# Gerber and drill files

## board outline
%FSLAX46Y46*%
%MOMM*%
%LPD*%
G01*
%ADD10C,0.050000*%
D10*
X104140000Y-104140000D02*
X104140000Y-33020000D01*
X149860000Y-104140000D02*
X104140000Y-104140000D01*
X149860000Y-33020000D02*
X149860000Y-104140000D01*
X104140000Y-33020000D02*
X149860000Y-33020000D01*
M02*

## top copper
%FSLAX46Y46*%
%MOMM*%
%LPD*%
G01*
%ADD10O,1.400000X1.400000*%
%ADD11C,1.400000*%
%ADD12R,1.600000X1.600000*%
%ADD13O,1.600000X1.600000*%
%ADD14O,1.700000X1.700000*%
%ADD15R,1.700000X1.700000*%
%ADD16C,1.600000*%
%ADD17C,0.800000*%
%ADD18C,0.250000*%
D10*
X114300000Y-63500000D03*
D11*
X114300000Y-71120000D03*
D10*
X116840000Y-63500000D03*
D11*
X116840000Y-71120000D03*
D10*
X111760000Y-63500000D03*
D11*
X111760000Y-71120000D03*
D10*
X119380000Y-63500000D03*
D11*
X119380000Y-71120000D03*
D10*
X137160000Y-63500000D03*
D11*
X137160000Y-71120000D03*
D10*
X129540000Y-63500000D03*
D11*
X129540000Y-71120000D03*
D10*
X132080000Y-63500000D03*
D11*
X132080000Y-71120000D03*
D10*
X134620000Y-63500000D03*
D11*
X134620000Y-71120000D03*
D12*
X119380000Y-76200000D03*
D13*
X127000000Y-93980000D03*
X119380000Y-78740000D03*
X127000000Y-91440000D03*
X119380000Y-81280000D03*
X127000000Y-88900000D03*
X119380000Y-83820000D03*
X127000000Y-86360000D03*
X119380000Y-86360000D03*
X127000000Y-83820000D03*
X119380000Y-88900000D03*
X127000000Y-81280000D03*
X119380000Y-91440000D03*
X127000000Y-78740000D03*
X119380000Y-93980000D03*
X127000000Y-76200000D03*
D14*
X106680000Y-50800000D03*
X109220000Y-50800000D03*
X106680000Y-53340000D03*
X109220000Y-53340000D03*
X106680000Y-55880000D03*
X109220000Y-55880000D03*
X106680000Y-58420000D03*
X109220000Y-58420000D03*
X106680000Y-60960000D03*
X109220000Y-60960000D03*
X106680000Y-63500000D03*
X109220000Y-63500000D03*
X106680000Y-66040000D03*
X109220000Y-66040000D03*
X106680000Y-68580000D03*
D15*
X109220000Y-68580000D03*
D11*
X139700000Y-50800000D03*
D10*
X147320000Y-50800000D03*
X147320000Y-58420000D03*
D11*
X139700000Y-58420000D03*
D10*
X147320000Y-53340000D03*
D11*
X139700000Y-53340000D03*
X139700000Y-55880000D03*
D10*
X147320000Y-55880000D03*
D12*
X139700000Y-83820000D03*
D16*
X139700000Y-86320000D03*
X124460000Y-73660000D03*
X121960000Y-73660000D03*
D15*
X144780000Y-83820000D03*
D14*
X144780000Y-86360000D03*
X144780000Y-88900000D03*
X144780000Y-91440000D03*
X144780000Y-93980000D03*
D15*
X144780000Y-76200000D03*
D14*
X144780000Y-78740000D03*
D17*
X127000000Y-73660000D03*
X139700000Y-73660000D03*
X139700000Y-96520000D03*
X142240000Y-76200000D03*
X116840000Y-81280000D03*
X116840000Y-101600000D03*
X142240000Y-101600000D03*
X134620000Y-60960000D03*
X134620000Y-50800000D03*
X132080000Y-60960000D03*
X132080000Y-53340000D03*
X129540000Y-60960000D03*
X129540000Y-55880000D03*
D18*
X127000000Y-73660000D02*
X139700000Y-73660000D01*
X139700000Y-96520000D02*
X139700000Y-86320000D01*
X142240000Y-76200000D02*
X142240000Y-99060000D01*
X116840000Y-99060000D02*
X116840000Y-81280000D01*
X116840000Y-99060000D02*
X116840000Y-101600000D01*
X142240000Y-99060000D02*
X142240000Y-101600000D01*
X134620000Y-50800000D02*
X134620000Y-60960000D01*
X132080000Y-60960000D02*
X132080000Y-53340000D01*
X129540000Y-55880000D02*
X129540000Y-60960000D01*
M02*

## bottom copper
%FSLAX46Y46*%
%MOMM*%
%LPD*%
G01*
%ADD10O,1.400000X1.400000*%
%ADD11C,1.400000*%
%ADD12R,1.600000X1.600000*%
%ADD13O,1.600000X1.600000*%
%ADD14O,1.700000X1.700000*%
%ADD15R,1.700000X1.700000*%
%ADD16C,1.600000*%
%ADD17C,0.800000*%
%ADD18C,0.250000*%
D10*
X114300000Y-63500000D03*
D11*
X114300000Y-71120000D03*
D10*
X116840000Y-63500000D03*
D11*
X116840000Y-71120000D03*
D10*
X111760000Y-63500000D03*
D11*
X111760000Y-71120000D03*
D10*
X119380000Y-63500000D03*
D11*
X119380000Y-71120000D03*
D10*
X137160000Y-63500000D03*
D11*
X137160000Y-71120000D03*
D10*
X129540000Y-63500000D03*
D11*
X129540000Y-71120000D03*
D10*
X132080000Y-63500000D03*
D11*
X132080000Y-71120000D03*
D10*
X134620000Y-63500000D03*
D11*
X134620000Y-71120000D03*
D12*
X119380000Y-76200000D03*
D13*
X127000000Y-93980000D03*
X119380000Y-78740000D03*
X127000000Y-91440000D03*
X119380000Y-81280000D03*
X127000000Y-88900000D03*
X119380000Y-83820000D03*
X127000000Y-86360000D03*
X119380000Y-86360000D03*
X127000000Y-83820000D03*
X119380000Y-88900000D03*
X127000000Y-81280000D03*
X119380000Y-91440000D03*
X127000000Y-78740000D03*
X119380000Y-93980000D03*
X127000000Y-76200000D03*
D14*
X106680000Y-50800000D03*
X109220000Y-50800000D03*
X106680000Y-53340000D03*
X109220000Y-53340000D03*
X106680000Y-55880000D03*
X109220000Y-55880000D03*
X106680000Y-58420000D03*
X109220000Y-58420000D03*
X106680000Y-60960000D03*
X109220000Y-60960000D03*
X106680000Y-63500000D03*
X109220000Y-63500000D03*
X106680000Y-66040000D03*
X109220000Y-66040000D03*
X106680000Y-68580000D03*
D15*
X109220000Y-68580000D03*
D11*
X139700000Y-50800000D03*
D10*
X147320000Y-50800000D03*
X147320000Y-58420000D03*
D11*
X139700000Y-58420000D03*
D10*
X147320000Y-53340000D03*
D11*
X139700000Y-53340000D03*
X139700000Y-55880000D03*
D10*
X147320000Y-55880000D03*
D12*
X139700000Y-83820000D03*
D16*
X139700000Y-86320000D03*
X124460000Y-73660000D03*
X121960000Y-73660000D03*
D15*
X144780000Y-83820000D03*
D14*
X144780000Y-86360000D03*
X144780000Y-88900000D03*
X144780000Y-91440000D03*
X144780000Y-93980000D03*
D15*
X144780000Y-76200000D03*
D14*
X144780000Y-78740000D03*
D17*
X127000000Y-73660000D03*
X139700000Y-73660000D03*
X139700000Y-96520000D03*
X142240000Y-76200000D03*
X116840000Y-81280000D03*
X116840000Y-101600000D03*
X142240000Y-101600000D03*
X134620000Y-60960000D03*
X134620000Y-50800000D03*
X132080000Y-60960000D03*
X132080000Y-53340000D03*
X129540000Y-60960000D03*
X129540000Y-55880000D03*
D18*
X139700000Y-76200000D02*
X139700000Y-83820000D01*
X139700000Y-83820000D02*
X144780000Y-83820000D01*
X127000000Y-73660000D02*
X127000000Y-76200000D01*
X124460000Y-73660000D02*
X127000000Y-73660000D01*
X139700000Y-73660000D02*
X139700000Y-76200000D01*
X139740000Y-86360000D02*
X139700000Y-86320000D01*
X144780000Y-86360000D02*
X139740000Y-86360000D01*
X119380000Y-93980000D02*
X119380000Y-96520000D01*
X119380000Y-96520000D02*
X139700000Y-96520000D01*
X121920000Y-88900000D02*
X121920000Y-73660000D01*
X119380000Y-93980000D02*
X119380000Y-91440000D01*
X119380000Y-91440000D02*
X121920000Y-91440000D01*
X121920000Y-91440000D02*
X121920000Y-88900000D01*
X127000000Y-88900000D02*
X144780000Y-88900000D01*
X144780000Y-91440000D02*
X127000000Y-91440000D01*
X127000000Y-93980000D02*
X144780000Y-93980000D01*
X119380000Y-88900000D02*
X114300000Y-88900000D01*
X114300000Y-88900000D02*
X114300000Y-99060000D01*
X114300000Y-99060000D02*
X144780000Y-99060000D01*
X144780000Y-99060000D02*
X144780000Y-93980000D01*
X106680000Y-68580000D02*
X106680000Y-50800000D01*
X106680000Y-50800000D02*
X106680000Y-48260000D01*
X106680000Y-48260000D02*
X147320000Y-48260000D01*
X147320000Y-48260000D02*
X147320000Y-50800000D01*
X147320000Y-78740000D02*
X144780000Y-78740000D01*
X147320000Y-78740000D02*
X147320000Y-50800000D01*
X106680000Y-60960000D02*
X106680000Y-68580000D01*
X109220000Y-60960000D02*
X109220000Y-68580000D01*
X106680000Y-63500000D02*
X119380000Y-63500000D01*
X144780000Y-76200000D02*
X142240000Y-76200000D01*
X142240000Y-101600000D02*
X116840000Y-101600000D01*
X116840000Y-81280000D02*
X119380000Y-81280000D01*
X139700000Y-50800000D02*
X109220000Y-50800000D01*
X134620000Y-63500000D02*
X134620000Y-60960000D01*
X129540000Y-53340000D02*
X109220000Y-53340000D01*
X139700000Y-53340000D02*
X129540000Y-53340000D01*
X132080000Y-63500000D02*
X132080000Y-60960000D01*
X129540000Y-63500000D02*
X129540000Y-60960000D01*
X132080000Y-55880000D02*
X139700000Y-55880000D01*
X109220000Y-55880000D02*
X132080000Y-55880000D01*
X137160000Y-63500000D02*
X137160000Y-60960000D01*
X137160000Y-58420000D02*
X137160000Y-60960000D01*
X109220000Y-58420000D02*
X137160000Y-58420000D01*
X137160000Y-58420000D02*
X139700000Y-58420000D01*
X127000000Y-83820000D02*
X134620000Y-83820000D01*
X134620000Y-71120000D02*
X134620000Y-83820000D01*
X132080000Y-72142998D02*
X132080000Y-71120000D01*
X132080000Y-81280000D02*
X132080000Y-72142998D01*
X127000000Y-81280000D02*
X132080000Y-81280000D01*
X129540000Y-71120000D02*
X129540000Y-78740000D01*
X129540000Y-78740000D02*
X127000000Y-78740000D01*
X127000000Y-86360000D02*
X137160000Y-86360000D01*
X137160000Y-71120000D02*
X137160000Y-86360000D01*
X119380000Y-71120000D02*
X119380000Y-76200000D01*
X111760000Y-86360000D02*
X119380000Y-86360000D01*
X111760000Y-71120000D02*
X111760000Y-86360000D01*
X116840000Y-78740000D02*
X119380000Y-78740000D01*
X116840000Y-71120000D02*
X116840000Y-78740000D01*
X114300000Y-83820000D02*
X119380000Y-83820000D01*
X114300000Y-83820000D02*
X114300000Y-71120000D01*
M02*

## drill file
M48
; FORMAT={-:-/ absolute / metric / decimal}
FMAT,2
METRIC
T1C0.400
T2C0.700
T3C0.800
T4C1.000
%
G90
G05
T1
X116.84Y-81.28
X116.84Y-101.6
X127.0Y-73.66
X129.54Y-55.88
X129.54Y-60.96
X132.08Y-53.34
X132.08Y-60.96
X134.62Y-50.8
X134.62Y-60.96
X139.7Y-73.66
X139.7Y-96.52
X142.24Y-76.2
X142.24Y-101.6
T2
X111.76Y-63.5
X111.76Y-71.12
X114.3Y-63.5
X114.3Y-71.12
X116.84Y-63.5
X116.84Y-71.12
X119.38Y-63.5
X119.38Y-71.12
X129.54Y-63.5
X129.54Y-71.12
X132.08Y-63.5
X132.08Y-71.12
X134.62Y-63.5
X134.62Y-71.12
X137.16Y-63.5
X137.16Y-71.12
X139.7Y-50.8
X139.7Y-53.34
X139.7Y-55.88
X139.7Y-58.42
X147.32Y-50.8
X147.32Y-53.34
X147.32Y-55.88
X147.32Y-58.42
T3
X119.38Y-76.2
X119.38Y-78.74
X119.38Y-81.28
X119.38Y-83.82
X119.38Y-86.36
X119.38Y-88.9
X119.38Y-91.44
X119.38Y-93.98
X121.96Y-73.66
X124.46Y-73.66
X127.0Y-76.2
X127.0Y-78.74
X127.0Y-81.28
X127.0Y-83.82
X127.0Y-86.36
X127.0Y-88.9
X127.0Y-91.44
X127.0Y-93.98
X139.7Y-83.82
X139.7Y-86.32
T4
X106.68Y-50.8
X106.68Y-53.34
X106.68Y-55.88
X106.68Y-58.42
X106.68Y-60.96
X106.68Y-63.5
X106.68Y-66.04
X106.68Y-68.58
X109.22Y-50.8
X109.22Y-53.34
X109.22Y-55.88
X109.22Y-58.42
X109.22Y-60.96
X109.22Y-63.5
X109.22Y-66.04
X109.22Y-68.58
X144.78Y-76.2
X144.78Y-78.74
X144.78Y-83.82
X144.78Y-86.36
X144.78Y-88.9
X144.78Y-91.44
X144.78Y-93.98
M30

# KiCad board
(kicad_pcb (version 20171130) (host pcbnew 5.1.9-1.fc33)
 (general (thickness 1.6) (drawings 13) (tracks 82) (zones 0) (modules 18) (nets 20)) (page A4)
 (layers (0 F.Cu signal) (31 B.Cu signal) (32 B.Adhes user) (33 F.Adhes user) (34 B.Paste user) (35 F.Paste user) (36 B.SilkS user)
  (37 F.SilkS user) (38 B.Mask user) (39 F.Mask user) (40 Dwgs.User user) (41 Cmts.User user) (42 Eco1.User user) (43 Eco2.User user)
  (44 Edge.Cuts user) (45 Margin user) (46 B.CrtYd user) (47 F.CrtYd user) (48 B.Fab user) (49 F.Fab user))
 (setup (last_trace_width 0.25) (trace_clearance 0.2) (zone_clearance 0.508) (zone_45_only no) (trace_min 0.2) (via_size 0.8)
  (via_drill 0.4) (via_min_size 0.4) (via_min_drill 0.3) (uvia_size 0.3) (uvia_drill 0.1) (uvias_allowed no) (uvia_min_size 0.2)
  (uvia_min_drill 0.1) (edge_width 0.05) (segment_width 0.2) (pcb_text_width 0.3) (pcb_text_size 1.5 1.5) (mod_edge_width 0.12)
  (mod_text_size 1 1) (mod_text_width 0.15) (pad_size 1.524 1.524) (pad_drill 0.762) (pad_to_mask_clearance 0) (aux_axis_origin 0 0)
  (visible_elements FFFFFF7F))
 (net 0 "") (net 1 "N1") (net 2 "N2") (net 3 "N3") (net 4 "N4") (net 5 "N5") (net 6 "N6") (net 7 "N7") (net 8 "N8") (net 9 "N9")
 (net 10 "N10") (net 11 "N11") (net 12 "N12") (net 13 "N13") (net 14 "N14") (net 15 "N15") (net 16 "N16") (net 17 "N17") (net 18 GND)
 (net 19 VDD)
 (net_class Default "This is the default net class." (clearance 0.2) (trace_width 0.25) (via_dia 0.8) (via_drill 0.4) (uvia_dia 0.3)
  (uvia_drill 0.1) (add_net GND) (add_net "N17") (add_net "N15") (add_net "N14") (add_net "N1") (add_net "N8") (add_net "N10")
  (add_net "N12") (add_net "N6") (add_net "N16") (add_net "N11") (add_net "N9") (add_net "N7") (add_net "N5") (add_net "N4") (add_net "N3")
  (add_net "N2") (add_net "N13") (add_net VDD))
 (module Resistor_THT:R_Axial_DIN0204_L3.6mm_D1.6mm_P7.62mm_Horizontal (layer F.Cu) (at 114.3 71.12 90)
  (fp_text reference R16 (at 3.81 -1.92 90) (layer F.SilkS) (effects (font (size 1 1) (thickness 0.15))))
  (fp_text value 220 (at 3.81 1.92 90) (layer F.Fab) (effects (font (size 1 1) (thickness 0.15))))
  (pad 2 thru_hole oval (at 7.62 0 90) (size 1.4 1.4) (drill 0.7) (layers *.Cu *.Mask) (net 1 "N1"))
  (pad 1 thru_hole circle (at 0 0 90) (size 1.4 1.4) (drill 0.7) (layers *.Cu *.Mask) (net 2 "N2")))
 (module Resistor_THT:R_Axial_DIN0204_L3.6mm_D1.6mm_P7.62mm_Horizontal (layer F.Cu) (at 116.84 71.12 90)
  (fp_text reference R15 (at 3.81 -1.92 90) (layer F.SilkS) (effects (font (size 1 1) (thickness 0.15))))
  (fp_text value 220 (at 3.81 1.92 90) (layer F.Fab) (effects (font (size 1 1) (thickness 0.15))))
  (pad 2 thru_hole oval (at 7.62 0 90) (size 1.4 1.4) (drill 0.7) (layers *.Cu *.Mask) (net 1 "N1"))
  (pad 1 thru_hole circle (at 0 0 90) (size 1.4 1.4) (drill 0.7) (layers *.Cu *.Mask) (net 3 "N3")))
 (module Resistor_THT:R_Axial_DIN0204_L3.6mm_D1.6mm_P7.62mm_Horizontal (layer F.Cu) (at 111.76 71.12 90)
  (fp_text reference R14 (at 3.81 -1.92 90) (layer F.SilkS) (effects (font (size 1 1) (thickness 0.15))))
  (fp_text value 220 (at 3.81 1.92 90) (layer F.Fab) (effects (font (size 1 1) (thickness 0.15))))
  (pad 2 thru_hole oval (at 7.62 0 90) (size 1.4 1.4) (drill 0.7) (layers *.Cu *.Mask) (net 1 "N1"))
  (pad 1 thru_hole circle (at 0 0 90) (size 1.4 1.4) (drill 0.7) (layers *.Cu *.Mask) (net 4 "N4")))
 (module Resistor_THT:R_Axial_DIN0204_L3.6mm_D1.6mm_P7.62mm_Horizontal (layer F.Cu) (at 119.38 71.12 90)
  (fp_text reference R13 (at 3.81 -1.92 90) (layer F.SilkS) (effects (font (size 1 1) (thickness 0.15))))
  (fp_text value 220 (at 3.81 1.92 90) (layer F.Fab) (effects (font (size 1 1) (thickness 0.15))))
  (pad 2 thru_hole oval (at 7.62 0 90) (size 1.4 1.4) (drill 0.7) (layers *.Cu *.Mask) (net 1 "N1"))
  (pad 1 thru_hole circle (at 0 0 90) (size 1.4 1.4) (drill 0.7) (layers *.Cu *.Mask) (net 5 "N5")))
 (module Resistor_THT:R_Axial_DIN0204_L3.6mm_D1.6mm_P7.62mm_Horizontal (layer F.Cu) (at 137.16 71.12 90)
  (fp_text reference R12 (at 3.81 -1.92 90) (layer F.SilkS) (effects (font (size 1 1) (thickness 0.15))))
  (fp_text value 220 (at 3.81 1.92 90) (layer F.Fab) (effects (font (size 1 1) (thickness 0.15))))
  (pad 2 thru_hole oval (at 7.62 0 90) (size 1.4 1.4) (drill 0.7) (layers *.Cu *.Mask) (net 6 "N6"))
  (pad 1 thru_hole circle (at 0 0 90) (size 1.4 1.4) (drill 0.7) (layers *.Cu *.Mask) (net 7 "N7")))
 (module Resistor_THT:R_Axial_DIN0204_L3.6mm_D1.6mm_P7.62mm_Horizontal (layer F.Cu) (at 129.54 71.12 90)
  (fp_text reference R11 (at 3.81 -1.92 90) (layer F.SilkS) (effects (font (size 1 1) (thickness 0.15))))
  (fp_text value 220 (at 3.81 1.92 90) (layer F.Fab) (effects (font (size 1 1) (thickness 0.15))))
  (pad 2 thru_hole oval (at 7.62 0 90) (size 1.4 1.4) (drill 0.7) (layers *.Cu *.Mask) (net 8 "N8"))
  (pad 1 thru_hole circle (at 0 0 90) (size 1.4 1.4) (drill 0.7) (layers *.Cu *.Mask) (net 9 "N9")))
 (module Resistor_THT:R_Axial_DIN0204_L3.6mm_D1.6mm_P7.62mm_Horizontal (layer F.Cu) (at 132.08 71.12 90)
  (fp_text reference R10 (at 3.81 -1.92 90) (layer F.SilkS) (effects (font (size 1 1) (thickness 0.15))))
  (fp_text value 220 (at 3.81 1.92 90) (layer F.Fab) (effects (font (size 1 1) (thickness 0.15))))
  (pad 2 thru_hole oval (at 7.62 0 90) (size 1.4 1.4) (drill 0.7) (layers *.Cu *.Mask) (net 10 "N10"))
  (pad 1 thru_hole circle (at 0 0 90) (size 1.4 1.4) (drill 0.7) (layers *.Cu *.Mask) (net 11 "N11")))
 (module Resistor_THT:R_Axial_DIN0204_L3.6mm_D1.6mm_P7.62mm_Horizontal (layer F.Cu) (at 134.62 71.12 90)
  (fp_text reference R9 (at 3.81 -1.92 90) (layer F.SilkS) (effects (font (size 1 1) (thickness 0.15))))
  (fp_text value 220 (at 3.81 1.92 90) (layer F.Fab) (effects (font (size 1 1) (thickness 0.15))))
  (pad 2 thru_hole oval (at 7.62 0 90) (size 1.4 1.4) (drill 0.7) (layers *.Cu *.Mask) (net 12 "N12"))
  (pad 1 thru_hole circle (at 0 0 90) (size 1.4 1.4) (drill 0.7) (layers *.Cu *.Mask) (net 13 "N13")))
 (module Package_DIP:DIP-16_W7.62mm (layer F.Cu) (at 119.38 76.2)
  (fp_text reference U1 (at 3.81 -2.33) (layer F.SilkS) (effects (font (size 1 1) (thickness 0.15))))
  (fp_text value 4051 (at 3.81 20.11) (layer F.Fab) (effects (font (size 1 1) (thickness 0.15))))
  (pad 1 thru_hole rect (at 0 0) (size 1.6 1.6) (drill 0.8) (layers *.Cu *.Mask) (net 5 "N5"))
  (pad 9 thru_hole oval (at 7.62 17.78) (size 1.6 1.6) (drill 0.8) (layers *.Cu *.Mask) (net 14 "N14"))
  (pad 2 thru_hole oval (at 0 2.54) (size 1.6 1.6) (drill 0.8) (layers *.Cu *.Mask) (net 3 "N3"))
  (pad 10 thru_hole oval (at 7.62 15.24) (size 1.6 1.6) (drill 0.8) (layers *.Cu *.Mask) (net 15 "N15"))
  (pad 3 thru_hole oval (at 0 5.08) (size 1.6 1.6) (drill 0.8) (layers *.Cu *.Mask) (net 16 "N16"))
  (pad 11 thru_hole oval (at 7.62 12.7) (size 1.6 1.6) (drill 0.8) (layers *.Cu *.Mask) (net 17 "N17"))
  (pad 4 thru_hole oval (at 0 7.62) (size 1.6 1.6) (drill 0.8) (layers *.Cu *.Mask) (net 2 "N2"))
  (pad 12 thru_hole oval (at 7.62 10.16) (size 1.6 1.6) (drill 0.8) (layers *.Cu *.Mask) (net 7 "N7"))
  (pad 5 thru_hole oval (at 0 10.16) (size 1.6 1.6) (drill 0.8) (layers *.Cu *.Mask) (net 4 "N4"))
  (pad 13 thru_hole oval (at 7.62 7.62) (size 1.6 1.6) (drill 0.8) (layers *.Cu *.Mask) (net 13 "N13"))
  (pad 6 thru_hole oval (at 0 12.7) (size 1.6 1.6) (drill 0.8) (layers *.Cu *.Mask) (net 14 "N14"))
  (pad 14 thru_hole oval (at 7.62 5.08) (size 1.6 1.6) (drill 0.8) (layers *.Cu *.Mask) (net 11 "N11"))
  (pad 7 thru_hole oval (at 0 15.24) (size 1.6 1.6) (drill 0.8) (layers *.Cu *.Mask) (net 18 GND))
  (pad 15 thru_hole oval (at 7.62 2.54) (size 1.6 1.6) (drill 0.8) (layers *.Cu *.Mask) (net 9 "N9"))
  (pad 8 thru_hole oval (at 0 17.78) (size 1.6 1.6) (drill 0.8) (layers *.Cu *.Mask) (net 18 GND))
  (pad 16 thru_hole oval (at 7.62 0) (size 1.6 1.6) (drill 0.8) (layers *.Cu *.Mask) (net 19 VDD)))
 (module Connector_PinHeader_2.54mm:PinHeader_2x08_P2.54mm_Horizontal (layer F.Cu) (at 109.22 68.58 180)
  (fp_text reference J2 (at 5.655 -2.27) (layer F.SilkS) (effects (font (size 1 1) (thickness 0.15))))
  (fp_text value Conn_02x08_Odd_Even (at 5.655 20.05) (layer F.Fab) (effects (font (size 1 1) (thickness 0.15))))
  (pad 16 thru_hole oval (at 2.54 17.78 180) (size 1.7 1.7) (drill 1) (layers *.Cu *.Mask) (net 1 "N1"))
  (pad 15 thru_hole oval (at 0 17.78 180) (size 1.7 1.7) (drill 1) (layers *.Cu *.Mask) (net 12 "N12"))
  (pad 14 thru_hole oval (at 2.54 15.24 180) (size 1.7 1.7) (drill 1) (layers *.Cu *.Mask) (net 1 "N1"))
  (pad 13 thru_hole oval (at 0 15.24 180) (size 1.7 1.7) (drill 1) (layers *.Cu *.Mask) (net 10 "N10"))
  (pad 12 thru_hole oval (at 2.54 12.7 180) (size 1.7 1.7) (drill 1) (layers *.Cu *.Mask) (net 1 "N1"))
  (pad 11 thru_hole oval (at 0 12.7 180) (size 1.7 1.7) (drill 1) (layers *.Cu *.Mask) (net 8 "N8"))
  (pad 10 thru_hole oval (at 2.54 10.16 180) (size 1.7 1.7) (drill 1) (layers *.Cu *.Mask) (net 1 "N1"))
  (pad 9 thru_hole oval (at 0 10.16 180) (size 1.7 1.7) (drill 1) (layers *.Cu *.Mask) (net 6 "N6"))
  (pad 8 thru_hole oval (at 2.54 7.62 180) (size 1.7 1.7) (drill 1) (layers *.Cu *.Mask) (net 1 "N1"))
  (pad 7 thru_hole oval (at 0 7.62 180) (size 1.7 1.7) (drill 1) (layers *.Cu *.Mask) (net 1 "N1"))
  (pad 6 thru_hole oval (at 2.54 5.08 180) (size 1.7 1.7) (drill 1) (layers *.Cu *.Mask) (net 1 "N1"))
  (pad 5 thru_hole oval (at 0 5.08 180) (size 1.7 1.7) (drill 1) (layers *.Cu *.Mask) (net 1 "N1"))
  (pad 4 thru_hole oval (at 2.54 2.54 180) (size 1.7 1.7) (drill 1) (layers *.Cu *.Mask) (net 1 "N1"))
  (pad 3 thru_hole oval (at 0 2.54 180) (size 1.7 1.7) (drill 1) (layers *.Cu *.Mask) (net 1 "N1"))
  (pad 2 thru_hole oval (at 2.54 0 180) (size 1.7 1.7) (drill 1) (layers *.Cu *.Mask) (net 1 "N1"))
  (pad 1 thru_hole rect (at 0 0 180) (size 1.7 1.7) (drill 1) (layers *.Cu *.Mask) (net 1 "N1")))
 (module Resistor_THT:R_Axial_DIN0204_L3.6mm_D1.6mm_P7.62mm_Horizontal (layer F.Cu) (at 139.7 50.8)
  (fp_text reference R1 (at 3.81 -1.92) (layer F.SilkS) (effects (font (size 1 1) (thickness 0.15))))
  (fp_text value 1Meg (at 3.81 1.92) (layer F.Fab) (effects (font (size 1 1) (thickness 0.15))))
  (pad 1 thru_hole circle (at 0 0) (size 1.4 1.4) (drill 0.7) (layers *.Cu *.Mask) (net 12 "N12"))
  (pad 2 thru_hole oval (at 7.62 0) (size 1.4 1.4) (drill 0.7) (layers *.Cu *.Mask) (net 1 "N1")))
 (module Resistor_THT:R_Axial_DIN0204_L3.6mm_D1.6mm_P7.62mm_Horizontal (layer F.Cu) (at 139.7 58.42)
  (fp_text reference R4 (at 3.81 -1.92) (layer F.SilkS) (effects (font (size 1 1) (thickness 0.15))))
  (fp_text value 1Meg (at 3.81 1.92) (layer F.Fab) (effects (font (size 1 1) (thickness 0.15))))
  (pad 2 thru_hole oval (at 7.62 0) (size 1.4 1.4) (drill 0.7) (layers *.Cu *.Mask) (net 1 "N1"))
  (pad 1 thru_hole circle (at 0 0) (size 1.4 1.4) (drill 0.7) (layers *.Cu *.Mask) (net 6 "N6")))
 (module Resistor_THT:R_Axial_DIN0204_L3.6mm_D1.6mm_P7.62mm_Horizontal (layer F.Cu) (at 139.7 53.34)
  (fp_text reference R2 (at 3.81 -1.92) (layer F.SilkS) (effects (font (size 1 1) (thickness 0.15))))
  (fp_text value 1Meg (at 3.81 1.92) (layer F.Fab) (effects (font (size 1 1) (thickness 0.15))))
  (pad 2 thru_hole oval (at 7.62 0) (size 1.4 1.4) (drill 0.7) (layers *.Cu *.Mask) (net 1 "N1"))
  (pad 1 thru_hole circle (at 0 0) (size 1.4 1.4) (drill 0.7) (layers *.Cu *.Mask) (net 10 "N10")))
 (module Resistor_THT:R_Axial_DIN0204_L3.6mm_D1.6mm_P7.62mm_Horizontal (layer F.Cu) (at 139.7 55.88)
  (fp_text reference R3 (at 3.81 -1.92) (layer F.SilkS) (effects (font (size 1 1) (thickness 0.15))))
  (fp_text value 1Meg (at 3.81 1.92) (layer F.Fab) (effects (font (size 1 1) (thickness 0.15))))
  (pad 1 thru_hole circle (at 0 0) (size 1.4 1.4) (drill 0.7) (layers *.Cu *.Mask) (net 8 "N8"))
  (pad 2 thru_hole oval (at 7.62 0) (size 1.4 1.4) (drill 0.7) (layers *.Cu *.Mask) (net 1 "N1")))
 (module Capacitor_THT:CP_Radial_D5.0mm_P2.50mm (layer F.Cu) (at 139.7 83.82 270)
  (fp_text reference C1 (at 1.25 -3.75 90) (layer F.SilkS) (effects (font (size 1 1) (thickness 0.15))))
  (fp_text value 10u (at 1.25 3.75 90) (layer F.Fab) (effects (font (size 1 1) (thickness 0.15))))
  (pad 1 thru_hole rect (at 0 0 270) (size 1.6 1.6) (drill 0.8) (layers *.Cu *.Mask) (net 19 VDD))
  (pad 2 thru_hole circle (at 2.5 0 270) (size 1.6 1.6) (drill 0.8) (layers *.Cu *.Mask) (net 18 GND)))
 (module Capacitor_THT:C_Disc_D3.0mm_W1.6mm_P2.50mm (layer F.Cu) (at 124.46 73.66 180)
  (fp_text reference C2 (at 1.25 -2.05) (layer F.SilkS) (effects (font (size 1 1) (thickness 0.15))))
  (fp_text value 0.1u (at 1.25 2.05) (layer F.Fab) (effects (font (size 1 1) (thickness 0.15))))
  (pad 1 thru_hole circle (at 0 0 180) (size 1.6 1.6) (drill 0.8) (layers *.Cu *.Mask) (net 19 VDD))
  (pad 2 thru_hole circle (at 2.5 0 180) (size 1.6 1.6) (drill 0.8) (layers *.Cu *.Mask) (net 18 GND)))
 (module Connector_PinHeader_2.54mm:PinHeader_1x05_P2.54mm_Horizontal (layer F.Cu) (at 144.78 83.82)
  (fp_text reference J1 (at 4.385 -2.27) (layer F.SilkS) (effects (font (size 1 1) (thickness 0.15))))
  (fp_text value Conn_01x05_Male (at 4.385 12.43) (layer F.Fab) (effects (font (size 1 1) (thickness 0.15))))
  (pad 1 thru_hole rect (at 0 0) (size 1.7 1.7) (drill 1) (layers *.Cu *.Mask) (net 19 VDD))
  (pad 2 thru_hole oval (at 0 2.54) (size 1.7 1.7) (drill 1) (layers *.Cu *.Mask) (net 18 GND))
  (pad 3 thru_hole oval (at 0 5.08) (size 1.7 1.7) (drill 1) (layers *.Cu *.Mask) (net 17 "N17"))
  (pad 4 thru_hole oval (at 0 7.62) (size 1.7 1.7) (drill 1) (layers *.Cu *.Mask) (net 15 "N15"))
  (pad 5 thru_hole oval (at 0 10.16) (size 1.7 1.7) (drill 1) (layers *.Cu *.Mask) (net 14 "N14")))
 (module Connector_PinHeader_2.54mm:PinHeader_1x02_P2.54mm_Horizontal (layer F.Cu) (at 144.78 76.2)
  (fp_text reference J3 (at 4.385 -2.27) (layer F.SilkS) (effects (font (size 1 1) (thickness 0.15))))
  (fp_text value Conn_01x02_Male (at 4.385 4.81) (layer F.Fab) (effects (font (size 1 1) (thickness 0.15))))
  (pad 1 thru_hole rect (at 0 0) (size 1.7 1.7) (drill 1) (layers *.Cu *.Mask) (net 16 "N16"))
  (pad 2 thru_hole oval (at 0 2.54) (size 1.7 1.7) (drill 1) (layers *.Cu *.Mask) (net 1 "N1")))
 (gr_line (start 104.14 104.14) (end 104.14 33.02) (layer Edge.Cuts) (width 0.05))
 (gr_line (start 149.86 104.14) (end 104.14 104.14) (layer Edge.Cuts) (width 0.05))
 (gr_line (start 149.86 33.02) (end 149.86 104.14) (layer Edge.Cuts) (width 0.05))
 (gr_line (start 104.14 33.02) (end 149.86 33.02) (layer Edge.Cuts) (width 0.05))
 (segment (start 139.7 76.2) (end 139.7 83.82) (width 0.25) (layer B.Cu) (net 19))
 (segment (start 139.7 83.82) (end 144.78 83.82) (width 0.25) (layer B.Cu) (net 19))
 (segment (start 127 73.66) (end 127 76.2) (width 0.25) (layer B.Cu) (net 19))
 (via (at 127 73.66) (size 0.8) (drill 0.4) (layers F.Cu B.Cu) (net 19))
 (segment (start 124.46 73.66) (end 127 73.66) (width 0.25) (layer B.Cu) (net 19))
 (via (at 139.7 73.66) (size 0.8) (drill 0.4) (layers F.Cu B.Cu) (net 19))
 (segment (start 127 73.66) (end 139.7 73.66) (width 0.25) (layer F.Cu) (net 19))
 (segment (start 139.7 73.66) (end 139.7 76.2) (width 0.25) (layer B.Cu) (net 19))
 (segment (start 139.74 86.36) (end 139.7 86.32) (width 0.25) (layer B.Cu) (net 18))
 (segment (start 144.78 86.36) (end 139.74 86.36) (width 0.25) (layer B.Cu) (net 18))
 (segment (start 119.38 93.98) (end 119.38 96.52) (width 0.25) (layer B.Cu) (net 18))
 (via (at 139.7 96.52) (size 0.8) (drill 0.4) (layers F.Cu B.Cu) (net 18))
 (segment (start 119.38 96.52) (end 139.7 96.52) (width 0.25) (layer B.Cu) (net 18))
 (segment (start 139.7 96.52) (end 139.7 86.32) (width 0.25) (layer F.Cu) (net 18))
 (segment (start 121.92 88.9) (end 121.92 73.66) (width 0.25) (layer B.Cu) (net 18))
 (segment (start 119.38 93.98) (end 119.38 91.44) (width 0.25) (layer B.Cu) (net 18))
 (segment (start 119.38 91.44) (end 121.92 91.44) (width 0.25) (layer B.Cu) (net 18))
 (segment (start 121.92 91.44) (end 121.92 88.9) (width 0.25) (layer B.Cu) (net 18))
 (segment (start 127 88.9) (end 144.78 88.9) (width 0.25) (layer B.Cu) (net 17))
 (segment (start 144.78 91.44) (end 127 91.44) (width 0.25) (layer B.Cu) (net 15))
 (segment (start 127 93.98) (end 144.78 93.98) (width 0.25) (layer B.Cu) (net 14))
 (segment (start 119.38 88.9) (end 114.3 88.9) (width 0.25) (layer B.Cu) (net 14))
 (segment (start 114.3 88.9) (end 114.3 99.06) (width 0.25) (layer B.Cu) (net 14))
 (segment (start 114.3 99.06) (end 144.78 99.06) (width 0.25) (layer B.Cu) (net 14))
 (segment (start 144.78 99.06) (end 144.78 93.98) (width 0.25) (layer B.Cu) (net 14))
 (segment (start 106.68 68.58) (end 106.68 50.8) (width 0.25) (layer B.Cu) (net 1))
 (segment (start 106.68 50.8) (end 106.68 48.26) (width 0.25) (layer B.Cu) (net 1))
 (segment (start 106.68 48.26) (end 147.32 48.26) (width 0.25) (layer B.Cu) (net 1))
 (segment (start 147.32 48.26) (end 147.32 50.8) (width 0.25) (layer B.Cu) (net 1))
 (segment (start 147.32 78.74) (end 144.78 78.74) (width 0.25) (layer B.Cu) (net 1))
 (segment (start 147.32 78.74) (end 147.32 50.8) (width 0.25) (layer B.Cu) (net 1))
 (segment (start 106.68 60.96) (end 106.68 68.58) (width 0.25) (layer B.Cu) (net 1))
 (segment (start 109.22 60.96) (end 109.22 68.58) (width 0.25) (layer B.Cu) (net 1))
 (segment (start 106.68 63.5) (end 119.38 63.5) (width 0.25) (layer B.Cu) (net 1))
 (via (at 142.24 76.2) (size 0.8) (drill 0.4) (layers F.Cu B.Cu) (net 16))
 (segment (start 144.78 76.2) (end 142.24 76.2) (width 0.25) (layer B.Cu) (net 16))
 (segment (start 142.24 76.2) (end 142.24 99.06) (width 0.25) (layer F.Cu) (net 16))
 (segment (start 142.24 101.6) (end 116.84 101.6) (width 0.25) (layer B.Cu) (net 16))
 (via (at 116.84 81.28) (size 0.8) (drill 0.4) (layers F.Cu B.Cu) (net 16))
 (segment (start 116.84 99.06) (end 116.84 81.28) (width 0.25) (layer F.Cu) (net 16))
 (segment (start 116.84 81.28) (end 119.38 81.28) (width 0.25) (layer B.Cu) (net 16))
 (via (at 116.84 101.6) (size 0.8) (drill 0.4) (layers F.Cu B.Cu) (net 16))
 (segment (start 116.84 99.06) (end 116.84 101.6) (width 0.25) (layer F.Cu) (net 16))
 (via (at 142.24 101.6) (size 0.8) (drill 0.4) (layers F.Cu B.Cu) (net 16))
 (segment (start 142.24 99.06) (end 142.24 101.6) (width 0.25) (layer F.Cu) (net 16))
 (segment (start 139.7 50.8) (end 109.22 50.8) (width 0.25) (layer B.Cu) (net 12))
 (via (at 134.62 60.96) (size 0.8) (drill 0.4) (layers F.Cu B.Cu) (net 12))
 (segment (start 134.62 63.5) (end 134.62 60.96) (width 0.25) (layer B.Cu) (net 12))
 (via (at 134.62 50.8) (size 0.8) (drill 0.4) (layers F.Cu B.Cu) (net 12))
 (segment (start 134.62 50.8) (end 134.62 60.96) (width 0.25) (layer F.Cu) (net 12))
 (segment (start 129.54 53.34) (end 109.22 53.34) (width 0.25) (layer B.Cu) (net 10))
 (segment (start 139.7 53.34) (end 129.54 53.34) (width 0.25) (layer B.Cu) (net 10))
 (via (at 132.08 60.96) (size 0.8) (drill 0.4) (layers F.Cu B.Cu) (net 10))
 (segment (start 132.08 63.5) (end 132.08 60.96) (width 0.25) (layer B.Cu) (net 10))
 (via (at 132.08 53.34) (size 0.8) (drill 0.4) (layers F.Cu B.Cu) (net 10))
 (segment (start 132.08 60.96) (end 132.08 53.34) (width 0.25) (layer F.Cu) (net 10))
 (via (at 129.54 60.96) (size 0.8) (drill 0.4) (layers F.Cu B.Cu) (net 8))
 (segment (start 129.54 63.5) (end 129.54 60.96) (width 0.25) (layer B.Cu) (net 8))
 (segment (start 132.08 55.88) (end 139.7 55.88) (width 0.25) (layer B.Cu) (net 8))
 (segment (start 109.22 55.88) (end 132.08 55.88) (width 0.25) (layer B.Cu) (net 8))
 (via (at 129.54 55.88) (size 0.8) (drill 0.4) (layers F.Cu B.Cu) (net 8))
 (segment (start 129.54 55.88) (end 129.54 60.96) (width 0.25) (layer F.Cu) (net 8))
 (segment (start 137.16 63.5) (end 137.16 60.96) (width 0.25) (layer B.Cu) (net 6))
 (segment (start 137.16 58.42) (end 137.16 60.96) (width 0.25) (layer B.Cu) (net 6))
 (segment (start 109.22 58.42) (end 137.16 58.42) (width 0.25) (layer B.Cu) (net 6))
 (segment (start 137.16 58.42) (end 139.7 58.42) (width 0.25) (layer B.Cu) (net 6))
 (segment (start 127 83.82) (end 134.62 83.82) (width 0.25) (layer B.Cu) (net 13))
 (segment (start 134.62 71.12) (end 134.62 83.82) (width 0.25) (layer B.Cu) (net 13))
 (segment (start 132.08 72.142998) (end 132.08 71.12) (width 0.25) (layer B.Cu) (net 11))
 (segment (start 132.08 81.28) (end 132.08 72.142998) (width 0.25) (layer B.Cu) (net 11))
 (segment (start 127 81.28) (end 132.08 81.28) (width 0.25) (layer B.Cu) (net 11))
 (segment (start 129.54 71.12) (end 129.54 78.74) (width 0.25) (layer B.Cu) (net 9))
 (segment (start 129.54 78.74) (end 127 78.74) (width 0.25) (layer B.Cu) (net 9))
 (segment (start 127 86.36) (end 137.16 86.36) (width 0.25) (layer B.Cu) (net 7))
 (segment (start 137.16 71.12) (end 137.16 86.36) (width 0.25) (layer B.Cu) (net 7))
 (segment (start 119.38 71.12) (end 119.38 76.2) (width 0.25) (layer B.Cu) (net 5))
 (segment (start 111.76 86.36) (end 119.38 86.36) (width 0.25) (layer B.Cu) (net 4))
 (segment (start 111.76 71.12) (end 111.76 86.36) (width 0.25) (layer B.Cu) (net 4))
 (segment (start 116.84 78.74) (end 119.38 78.74) (width 0.25) (layer B.Cu) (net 3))
 (segment (start 116.84 71.12) (end 116.84 78.74) (width 0.25) (layer B.Cu) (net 3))
 (segment (start 114.3 83.82) (end 119.38 83.82) (width 0.25) (layer B.Cu) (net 2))
 (segment (start 114.3 83.82) (end 114.3 71.12) (width 0.25) (layer B.Cu) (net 2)))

